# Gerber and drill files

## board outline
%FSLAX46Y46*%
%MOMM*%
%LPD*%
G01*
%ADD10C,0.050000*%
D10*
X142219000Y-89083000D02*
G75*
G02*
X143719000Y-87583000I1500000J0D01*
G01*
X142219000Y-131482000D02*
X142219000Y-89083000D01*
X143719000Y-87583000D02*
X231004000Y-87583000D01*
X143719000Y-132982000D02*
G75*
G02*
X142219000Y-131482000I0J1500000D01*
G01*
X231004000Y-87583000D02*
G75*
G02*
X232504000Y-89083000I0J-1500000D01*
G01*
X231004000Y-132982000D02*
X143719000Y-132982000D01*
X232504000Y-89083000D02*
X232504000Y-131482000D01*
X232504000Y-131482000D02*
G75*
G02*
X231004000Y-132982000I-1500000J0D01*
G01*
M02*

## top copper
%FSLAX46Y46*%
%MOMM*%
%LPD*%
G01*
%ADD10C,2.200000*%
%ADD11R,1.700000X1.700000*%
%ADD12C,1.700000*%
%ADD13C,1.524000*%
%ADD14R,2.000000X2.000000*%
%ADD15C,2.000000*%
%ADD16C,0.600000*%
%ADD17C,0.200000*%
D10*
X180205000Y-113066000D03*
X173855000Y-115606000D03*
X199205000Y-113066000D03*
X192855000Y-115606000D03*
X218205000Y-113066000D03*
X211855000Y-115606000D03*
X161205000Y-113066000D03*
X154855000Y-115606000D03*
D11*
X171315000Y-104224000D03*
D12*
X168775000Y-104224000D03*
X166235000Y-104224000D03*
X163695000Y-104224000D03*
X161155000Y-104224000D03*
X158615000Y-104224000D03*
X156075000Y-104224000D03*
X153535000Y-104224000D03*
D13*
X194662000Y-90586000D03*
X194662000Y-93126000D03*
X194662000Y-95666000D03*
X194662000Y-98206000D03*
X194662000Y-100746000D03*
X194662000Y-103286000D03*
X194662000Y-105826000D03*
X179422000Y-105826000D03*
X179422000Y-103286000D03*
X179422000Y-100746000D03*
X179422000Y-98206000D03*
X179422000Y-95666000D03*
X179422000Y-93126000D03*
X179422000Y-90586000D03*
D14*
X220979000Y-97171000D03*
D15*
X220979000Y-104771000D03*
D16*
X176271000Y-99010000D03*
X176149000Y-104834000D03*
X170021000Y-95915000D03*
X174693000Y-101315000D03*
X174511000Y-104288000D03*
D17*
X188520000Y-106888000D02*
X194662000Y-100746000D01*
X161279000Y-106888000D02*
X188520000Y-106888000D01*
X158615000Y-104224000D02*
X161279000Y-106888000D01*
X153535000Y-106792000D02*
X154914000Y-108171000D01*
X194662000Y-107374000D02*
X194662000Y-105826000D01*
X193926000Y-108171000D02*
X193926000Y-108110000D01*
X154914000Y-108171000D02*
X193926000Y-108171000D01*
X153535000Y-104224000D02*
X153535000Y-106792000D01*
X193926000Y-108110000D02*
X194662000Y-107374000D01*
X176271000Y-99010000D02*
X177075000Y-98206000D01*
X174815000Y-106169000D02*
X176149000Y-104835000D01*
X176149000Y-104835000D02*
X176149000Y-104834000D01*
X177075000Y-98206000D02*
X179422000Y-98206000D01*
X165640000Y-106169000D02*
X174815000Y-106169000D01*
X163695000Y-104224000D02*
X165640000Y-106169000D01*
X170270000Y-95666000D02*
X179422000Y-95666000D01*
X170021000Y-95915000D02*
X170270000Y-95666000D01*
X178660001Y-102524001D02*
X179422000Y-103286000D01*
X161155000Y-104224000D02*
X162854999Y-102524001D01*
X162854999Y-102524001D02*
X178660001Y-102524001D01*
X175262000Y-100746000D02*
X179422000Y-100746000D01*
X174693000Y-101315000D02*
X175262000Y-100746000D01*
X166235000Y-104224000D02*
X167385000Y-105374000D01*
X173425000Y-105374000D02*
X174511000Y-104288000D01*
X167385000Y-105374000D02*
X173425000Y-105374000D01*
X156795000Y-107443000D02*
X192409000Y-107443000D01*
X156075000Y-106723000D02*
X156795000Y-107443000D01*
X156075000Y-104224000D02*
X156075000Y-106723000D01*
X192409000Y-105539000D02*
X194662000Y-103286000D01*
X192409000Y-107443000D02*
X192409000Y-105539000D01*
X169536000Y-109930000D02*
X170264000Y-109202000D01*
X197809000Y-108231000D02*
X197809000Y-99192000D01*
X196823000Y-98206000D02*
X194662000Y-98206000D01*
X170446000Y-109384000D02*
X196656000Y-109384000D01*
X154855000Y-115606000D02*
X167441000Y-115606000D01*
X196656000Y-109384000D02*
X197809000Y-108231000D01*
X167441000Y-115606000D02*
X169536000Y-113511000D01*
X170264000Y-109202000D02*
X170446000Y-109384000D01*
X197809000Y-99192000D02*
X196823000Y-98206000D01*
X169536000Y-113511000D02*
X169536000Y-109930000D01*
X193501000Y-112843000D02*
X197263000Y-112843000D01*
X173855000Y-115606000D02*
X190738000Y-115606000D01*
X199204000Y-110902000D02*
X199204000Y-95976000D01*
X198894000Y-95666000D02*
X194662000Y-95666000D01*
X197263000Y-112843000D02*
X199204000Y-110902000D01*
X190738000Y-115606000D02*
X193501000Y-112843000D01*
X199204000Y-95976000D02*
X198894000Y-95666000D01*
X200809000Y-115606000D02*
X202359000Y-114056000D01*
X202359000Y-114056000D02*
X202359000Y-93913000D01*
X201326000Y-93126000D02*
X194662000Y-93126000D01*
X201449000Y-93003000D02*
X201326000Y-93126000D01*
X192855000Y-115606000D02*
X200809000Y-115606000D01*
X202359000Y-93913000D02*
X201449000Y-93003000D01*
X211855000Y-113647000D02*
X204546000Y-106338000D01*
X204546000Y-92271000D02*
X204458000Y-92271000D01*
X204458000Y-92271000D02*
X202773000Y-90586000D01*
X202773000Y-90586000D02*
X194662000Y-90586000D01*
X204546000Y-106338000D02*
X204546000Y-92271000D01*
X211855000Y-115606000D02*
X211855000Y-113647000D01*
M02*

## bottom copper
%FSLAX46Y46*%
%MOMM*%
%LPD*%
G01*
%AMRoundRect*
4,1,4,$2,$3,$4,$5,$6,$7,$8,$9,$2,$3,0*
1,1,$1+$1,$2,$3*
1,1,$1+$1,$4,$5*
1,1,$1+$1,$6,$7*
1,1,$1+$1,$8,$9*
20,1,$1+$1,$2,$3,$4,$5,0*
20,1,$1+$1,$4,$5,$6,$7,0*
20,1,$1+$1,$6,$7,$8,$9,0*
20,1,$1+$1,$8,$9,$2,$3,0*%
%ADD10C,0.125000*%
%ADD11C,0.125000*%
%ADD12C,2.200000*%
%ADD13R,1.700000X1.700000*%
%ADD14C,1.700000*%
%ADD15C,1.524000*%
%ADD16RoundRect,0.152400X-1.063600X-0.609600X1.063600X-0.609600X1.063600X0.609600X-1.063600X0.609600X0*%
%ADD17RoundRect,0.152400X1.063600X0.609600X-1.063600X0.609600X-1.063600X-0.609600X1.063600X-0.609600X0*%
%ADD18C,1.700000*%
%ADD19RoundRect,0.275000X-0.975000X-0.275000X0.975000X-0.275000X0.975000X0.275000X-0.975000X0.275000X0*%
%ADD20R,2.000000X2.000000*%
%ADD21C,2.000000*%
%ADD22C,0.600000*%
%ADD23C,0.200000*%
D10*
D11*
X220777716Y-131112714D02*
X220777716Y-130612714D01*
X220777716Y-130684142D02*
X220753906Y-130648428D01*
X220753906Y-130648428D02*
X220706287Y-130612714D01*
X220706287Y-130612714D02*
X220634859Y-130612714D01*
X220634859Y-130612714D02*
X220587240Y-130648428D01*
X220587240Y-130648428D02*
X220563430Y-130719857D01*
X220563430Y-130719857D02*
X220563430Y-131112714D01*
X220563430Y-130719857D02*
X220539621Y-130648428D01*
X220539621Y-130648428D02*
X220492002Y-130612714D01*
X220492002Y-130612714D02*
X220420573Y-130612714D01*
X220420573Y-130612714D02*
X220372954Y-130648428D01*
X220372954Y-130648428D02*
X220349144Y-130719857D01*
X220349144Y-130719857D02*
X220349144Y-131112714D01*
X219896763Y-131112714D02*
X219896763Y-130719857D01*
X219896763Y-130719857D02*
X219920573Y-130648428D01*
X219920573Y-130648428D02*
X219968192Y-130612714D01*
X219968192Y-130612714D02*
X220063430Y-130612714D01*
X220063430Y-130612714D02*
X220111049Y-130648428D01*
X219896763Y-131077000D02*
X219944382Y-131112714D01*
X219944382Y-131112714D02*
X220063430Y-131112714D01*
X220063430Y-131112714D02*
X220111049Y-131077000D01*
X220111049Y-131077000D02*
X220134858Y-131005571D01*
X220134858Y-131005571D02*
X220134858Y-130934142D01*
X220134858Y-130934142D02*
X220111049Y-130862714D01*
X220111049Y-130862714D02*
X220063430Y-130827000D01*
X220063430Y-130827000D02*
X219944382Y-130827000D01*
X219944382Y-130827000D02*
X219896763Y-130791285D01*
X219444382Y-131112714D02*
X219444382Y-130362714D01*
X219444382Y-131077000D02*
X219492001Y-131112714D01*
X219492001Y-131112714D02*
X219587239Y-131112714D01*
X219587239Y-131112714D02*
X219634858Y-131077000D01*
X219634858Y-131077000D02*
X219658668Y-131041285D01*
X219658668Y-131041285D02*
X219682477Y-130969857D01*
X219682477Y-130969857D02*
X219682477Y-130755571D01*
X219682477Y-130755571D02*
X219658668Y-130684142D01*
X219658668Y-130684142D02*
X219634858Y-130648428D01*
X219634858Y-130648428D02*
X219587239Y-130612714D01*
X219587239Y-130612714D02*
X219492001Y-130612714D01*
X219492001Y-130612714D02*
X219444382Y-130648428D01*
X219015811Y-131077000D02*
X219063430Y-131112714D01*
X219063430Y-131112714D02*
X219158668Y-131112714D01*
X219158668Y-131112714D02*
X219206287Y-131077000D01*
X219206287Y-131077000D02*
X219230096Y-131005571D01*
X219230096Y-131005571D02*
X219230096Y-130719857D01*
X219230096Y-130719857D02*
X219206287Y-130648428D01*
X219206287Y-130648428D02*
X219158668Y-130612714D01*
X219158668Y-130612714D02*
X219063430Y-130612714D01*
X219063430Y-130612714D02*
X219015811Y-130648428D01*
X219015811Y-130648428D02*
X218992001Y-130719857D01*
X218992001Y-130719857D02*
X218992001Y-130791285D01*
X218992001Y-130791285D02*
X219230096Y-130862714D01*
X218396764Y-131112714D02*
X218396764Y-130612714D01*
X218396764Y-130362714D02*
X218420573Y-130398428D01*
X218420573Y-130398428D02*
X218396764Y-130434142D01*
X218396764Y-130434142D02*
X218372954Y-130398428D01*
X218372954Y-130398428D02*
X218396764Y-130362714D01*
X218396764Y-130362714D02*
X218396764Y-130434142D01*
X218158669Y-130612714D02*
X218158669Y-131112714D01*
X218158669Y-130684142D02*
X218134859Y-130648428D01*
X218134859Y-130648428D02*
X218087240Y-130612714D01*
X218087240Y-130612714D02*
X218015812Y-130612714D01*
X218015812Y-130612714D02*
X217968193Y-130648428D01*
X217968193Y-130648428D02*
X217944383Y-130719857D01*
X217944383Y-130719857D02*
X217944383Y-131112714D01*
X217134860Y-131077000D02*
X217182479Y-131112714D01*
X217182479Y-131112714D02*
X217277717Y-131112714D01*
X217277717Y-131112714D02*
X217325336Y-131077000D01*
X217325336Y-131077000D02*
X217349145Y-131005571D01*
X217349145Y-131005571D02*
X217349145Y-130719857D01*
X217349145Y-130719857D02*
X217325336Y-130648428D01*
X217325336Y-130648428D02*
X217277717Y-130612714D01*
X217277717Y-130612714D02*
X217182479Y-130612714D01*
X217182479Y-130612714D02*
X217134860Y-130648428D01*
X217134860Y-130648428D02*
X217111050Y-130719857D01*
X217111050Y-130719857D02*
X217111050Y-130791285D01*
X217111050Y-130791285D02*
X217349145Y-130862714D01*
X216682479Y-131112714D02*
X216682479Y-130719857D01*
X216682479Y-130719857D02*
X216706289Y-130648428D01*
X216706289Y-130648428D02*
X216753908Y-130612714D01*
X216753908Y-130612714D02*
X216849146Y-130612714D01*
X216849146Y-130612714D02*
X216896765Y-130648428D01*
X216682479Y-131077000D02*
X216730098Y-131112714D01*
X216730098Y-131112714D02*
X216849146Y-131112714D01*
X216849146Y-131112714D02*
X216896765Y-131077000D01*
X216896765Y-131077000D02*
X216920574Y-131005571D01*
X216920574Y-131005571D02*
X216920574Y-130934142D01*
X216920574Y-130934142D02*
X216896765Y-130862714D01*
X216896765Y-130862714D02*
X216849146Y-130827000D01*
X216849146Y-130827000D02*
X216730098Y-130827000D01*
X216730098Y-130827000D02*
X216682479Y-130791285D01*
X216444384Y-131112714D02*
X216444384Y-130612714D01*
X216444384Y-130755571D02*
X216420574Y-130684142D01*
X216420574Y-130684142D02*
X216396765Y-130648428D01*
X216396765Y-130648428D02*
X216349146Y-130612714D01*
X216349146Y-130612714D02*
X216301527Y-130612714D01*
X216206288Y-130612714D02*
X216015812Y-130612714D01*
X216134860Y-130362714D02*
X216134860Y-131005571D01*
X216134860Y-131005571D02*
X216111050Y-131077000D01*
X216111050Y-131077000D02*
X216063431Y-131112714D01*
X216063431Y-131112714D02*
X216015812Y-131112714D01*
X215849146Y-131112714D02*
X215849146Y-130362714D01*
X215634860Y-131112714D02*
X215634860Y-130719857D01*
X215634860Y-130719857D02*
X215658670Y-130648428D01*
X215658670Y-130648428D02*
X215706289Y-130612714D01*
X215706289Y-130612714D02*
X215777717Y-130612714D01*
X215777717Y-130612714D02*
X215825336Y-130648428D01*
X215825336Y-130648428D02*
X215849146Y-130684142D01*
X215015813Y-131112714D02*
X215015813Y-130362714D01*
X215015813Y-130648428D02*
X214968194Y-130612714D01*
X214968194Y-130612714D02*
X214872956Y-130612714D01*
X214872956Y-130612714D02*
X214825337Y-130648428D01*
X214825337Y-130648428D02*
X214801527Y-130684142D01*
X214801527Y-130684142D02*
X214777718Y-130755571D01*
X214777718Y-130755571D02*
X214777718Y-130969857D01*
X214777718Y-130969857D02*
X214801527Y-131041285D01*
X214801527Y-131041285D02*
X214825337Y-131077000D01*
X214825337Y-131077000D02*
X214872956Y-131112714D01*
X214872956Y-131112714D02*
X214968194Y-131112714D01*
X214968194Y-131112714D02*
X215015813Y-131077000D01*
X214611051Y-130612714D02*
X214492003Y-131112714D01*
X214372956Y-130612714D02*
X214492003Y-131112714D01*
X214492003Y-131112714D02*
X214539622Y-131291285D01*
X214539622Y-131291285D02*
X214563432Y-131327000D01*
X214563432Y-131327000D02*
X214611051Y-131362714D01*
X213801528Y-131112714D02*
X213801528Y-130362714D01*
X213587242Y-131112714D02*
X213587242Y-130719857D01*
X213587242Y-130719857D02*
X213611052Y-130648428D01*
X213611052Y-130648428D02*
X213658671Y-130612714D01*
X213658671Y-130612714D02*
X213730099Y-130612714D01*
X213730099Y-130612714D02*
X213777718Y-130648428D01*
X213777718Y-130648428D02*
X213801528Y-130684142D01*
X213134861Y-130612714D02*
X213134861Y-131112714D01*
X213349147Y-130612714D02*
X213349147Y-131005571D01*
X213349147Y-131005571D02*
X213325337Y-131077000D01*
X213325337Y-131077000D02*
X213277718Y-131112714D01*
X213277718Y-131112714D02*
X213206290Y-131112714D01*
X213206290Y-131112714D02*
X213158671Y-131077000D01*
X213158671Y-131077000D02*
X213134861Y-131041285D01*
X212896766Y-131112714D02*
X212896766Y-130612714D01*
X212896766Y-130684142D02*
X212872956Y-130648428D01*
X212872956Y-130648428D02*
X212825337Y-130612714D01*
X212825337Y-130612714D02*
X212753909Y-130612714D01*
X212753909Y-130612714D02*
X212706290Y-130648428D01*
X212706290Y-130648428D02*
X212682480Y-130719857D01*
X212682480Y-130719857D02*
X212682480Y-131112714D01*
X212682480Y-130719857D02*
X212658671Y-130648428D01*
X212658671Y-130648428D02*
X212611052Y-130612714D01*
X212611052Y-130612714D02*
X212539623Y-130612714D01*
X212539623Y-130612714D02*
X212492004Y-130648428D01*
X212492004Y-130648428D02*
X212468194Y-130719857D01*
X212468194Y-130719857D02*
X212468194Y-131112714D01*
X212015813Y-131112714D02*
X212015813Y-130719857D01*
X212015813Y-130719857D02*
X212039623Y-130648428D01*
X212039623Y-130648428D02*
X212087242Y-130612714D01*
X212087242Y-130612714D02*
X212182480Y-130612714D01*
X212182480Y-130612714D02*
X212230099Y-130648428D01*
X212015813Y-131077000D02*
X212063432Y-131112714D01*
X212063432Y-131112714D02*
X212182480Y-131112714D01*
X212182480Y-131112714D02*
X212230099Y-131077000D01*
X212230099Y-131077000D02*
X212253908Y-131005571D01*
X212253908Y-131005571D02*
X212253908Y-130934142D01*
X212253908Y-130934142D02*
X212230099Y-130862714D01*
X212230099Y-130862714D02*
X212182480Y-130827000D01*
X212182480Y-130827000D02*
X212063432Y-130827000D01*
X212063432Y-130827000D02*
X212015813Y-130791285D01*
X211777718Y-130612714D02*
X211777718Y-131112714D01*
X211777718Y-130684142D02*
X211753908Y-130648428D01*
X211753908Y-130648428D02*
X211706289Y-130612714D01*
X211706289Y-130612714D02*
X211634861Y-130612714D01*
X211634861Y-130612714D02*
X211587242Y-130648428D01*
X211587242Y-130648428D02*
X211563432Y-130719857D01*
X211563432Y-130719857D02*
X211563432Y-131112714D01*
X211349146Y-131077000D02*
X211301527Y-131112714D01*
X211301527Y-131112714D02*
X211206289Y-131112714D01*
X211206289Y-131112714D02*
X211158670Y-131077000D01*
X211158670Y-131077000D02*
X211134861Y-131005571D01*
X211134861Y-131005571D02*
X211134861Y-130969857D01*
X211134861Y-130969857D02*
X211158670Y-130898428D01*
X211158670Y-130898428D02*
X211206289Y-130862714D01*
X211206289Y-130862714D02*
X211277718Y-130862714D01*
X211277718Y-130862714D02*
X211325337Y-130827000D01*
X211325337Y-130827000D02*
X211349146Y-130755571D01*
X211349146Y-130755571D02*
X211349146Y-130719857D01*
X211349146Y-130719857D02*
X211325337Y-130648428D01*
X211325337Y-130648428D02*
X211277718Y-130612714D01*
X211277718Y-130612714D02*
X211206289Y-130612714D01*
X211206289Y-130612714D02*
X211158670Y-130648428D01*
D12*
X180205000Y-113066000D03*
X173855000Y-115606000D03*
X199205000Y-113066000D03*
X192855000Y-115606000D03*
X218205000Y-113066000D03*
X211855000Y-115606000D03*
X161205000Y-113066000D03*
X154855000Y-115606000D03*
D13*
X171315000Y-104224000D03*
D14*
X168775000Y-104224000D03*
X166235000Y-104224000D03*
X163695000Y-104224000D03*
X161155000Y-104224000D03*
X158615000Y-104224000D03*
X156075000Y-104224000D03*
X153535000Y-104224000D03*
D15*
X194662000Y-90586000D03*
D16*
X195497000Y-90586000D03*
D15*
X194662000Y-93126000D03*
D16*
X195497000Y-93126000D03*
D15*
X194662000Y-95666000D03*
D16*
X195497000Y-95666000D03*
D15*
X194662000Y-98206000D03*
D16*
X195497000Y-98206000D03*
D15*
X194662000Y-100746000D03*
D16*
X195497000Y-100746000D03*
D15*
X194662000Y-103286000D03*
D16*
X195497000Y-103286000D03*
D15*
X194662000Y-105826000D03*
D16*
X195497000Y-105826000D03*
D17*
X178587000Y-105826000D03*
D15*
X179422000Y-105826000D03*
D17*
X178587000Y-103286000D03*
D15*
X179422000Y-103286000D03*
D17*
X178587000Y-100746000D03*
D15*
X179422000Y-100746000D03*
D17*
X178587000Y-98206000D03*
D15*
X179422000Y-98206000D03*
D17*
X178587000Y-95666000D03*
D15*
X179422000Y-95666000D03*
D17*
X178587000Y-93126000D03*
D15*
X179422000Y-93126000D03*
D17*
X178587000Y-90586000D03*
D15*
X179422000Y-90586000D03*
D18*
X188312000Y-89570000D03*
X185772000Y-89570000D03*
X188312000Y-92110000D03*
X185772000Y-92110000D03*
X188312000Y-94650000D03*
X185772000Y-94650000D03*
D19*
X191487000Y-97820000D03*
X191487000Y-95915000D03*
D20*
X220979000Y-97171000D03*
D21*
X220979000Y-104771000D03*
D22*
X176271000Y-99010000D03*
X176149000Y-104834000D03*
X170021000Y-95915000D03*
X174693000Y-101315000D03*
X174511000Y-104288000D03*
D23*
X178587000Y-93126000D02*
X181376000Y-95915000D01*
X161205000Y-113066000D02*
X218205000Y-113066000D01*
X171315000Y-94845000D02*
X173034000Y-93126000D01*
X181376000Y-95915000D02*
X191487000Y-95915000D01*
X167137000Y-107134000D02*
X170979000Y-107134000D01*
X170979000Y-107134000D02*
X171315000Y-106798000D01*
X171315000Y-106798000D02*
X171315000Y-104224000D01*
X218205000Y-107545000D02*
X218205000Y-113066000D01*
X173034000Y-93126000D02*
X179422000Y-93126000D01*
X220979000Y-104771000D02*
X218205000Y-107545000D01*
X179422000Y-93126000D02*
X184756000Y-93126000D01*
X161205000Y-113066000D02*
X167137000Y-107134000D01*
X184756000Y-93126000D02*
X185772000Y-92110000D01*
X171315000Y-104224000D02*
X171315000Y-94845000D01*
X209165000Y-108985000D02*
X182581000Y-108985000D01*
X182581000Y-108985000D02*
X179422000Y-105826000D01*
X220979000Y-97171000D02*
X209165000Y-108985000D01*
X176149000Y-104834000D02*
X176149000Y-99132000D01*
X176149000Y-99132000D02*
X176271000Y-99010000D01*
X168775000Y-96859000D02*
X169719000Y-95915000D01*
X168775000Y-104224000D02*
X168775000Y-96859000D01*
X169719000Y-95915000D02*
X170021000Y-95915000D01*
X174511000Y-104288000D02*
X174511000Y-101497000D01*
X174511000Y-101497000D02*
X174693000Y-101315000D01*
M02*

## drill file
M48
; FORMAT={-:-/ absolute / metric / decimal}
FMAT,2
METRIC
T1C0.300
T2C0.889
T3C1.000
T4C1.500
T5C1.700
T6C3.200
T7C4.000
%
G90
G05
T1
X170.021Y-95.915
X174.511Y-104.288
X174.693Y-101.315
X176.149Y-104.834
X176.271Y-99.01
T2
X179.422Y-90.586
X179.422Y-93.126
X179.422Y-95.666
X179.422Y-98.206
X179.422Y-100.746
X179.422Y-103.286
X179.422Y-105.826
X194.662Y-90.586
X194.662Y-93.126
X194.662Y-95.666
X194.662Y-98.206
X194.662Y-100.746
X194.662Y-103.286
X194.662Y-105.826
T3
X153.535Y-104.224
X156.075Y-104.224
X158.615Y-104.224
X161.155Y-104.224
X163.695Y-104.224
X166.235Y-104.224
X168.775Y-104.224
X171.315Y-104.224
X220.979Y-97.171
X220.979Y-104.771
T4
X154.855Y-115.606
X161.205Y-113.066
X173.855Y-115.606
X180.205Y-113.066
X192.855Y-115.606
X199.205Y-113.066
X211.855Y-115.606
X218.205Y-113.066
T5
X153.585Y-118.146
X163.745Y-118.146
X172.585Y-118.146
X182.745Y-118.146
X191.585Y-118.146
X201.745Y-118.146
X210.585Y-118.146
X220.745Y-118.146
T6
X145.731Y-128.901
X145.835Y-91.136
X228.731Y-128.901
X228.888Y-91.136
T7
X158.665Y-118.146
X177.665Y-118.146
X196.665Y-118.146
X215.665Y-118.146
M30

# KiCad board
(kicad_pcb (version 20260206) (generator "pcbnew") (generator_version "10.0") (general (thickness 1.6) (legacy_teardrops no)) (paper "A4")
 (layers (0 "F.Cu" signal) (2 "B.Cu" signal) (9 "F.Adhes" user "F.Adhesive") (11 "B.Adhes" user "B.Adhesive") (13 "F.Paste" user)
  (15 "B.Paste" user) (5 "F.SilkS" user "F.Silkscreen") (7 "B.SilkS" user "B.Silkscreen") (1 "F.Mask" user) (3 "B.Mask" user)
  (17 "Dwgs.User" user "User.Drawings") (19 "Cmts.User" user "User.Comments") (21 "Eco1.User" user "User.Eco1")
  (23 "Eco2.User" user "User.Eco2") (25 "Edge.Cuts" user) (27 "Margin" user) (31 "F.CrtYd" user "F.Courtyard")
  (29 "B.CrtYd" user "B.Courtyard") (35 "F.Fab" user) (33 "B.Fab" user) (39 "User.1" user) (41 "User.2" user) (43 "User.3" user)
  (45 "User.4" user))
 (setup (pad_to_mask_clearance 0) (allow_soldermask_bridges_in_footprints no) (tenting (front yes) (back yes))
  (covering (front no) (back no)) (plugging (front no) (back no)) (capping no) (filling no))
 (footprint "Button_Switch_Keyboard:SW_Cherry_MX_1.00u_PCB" (layer "F.Cu") (at 180.205 113.066)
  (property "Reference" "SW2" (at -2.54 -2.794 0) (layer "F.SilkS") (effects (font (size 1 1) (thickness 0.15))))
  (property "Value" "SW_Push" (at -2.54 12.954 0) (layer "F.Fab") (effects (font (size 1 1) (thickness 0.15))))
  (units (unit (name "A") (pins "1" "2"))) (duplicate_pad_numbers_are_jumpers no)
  (pad "" np_thru_hole circle (at -7.62 5.08) (size 1.7 1.7) (drill 1.7) (layers "*.Cu" "*.Mask"))
  (pad "" np_thru_hole circle (at -2.54 5.08) (size 4 4) (drill 4) (layers "*.Cu" "*.Mask"))
  (pad "" np_thru_hole circle (at 2.54 5.08) (size 1.7 1.7) (drill 1.7) (layers "*.Cu" "*.Mask"))
  (pad "1" thru_hole circle (at 0 0) (size 2.2 2.2) (drill 1.5) (layers "*.Cu" "*.Mask") (remove_unused_layers no) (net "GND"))
  (pad "2" thru_hole circle (at -6.35 2.54) (size 2.2 2.2) (drill 1.5) (layers "*.Cu" "*.Mask") (remove_unused_layers no)
   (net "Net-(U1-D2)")))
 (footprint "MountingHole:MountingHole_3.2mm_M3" (layer "F.Cu") (at 228.888 91.136)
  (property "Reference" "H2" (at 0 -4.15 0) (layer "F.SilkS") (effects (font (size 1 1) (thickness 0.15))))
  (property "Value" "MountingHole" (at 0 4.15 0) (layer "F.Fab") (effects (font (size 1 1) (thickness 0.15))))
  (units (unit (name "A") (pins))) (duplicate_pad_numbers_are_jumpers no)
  (pad "" np_thru_hole circle (at 0 0) (size 3.2 3.2) (drill 3.2) (layers "*.Cu" "*.Mask")))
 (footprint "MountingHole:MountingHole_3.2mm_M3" (layer "F.Cu") (at 145.731 128.901)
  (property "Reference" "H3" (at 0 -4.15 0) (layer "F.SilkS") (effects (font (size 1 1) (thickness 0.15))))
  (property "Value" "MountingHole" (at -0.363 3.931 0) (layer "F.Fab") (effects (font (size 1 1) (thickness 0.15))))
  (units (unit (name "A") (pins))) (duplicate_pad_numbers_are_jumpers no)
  (pad "" np_thru_hole circle (at 0 0) (size 3.2 3.2) (drill 3.2) (layers "*.Cu" "*.Mask")))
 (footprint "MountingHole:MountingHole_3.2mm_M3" (layer "F.Cu") (at 228.731 128.901)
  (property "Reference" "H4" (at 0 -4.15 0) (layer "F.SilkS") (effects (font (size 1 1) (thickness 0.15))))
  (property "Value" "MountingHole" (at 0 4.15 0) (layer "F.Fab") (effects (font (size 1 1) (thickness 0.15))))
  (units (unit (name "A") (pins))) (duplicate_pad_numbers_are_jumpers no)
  (pad "" np_thru_hole circle (at 0 0) (size 3.2 3.2) (drill 3.2) (layers "*.Cu" "*.Mask")))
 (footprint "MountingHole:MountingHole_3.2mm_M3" (layer "F.Cu") (at 145.835 91.136)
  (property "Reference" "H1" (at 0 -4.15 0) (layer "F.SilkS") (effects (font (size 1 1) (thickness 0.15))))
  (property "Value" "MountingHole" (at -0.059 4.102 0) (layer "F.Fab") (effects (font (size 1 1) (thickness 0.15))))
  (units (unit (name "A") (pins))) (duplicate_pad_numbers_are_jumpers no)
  (pad "" np_thru_hole circle (at 0 0) (size 3.2 3.2) (drill 3.2) (layers "*.Cu" "*.Mask")))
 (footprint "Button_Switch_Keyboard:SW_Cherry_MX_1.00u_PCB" (layer "F.Cu") (at 199.205 113.066)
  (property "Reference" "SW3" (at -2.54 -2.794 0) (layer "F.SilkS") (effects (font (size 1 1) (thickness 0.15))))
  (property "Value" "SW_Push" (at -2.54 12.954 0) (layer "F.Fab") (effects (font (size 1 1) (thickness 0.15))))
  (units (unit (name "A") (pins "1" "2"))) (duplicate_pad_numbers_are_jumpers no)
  (pad "" np_thru_hole circle (at -7.62 5.08) (size 1.7 1.7) (drill 1.7) (layers "*.Cu" "*.Mask"))
  (pad "" np_thru_hole circle (at -2.54 5.08) (size 4 4) (drill 4) (layers "*.Cu" "*.Mask"))
  (pad "" np_thru_hole circle (at 2.54 5.08) (size 1.7 1.7) (drill 1.7) (layers "*.Cu" "*.Mask"))
  (pad "1" thru_hole circle (at 0 0) (size 2.2 2.2) (drill 1.5) (layers "*.Cu" "*.Mask") (remove_unused_layers no) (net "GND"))
  (pad "2" thru_hole circle (at -6.35 2.54) (size 2.2 2.2) (drill 1.5) (layers "*.Cu" "*.Mask") (remove_unused_layers no)
   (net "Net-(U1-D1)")))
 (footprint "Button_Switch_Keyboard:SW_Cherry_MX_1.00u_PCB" (layer "F.Cu") (at 218.205 113.066)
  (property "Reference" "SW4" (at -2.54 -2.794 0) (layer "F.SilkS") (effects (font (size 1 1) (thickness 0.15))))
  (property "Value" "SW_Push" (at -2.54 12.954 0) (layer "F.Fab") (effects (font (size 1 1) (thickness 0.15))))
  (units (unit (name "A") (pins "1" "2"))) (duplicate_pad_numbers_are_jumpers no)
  (pad "" np_thru_hole circle (at -7.62 5.08) (size 1.7 1.7) (drill 1.7) (layers "*.Cu" "*.Mask"))
  (pad "" np_thru_hole circle (at -2.54 5.08) (size 4 4) (drill 4) (layers "*.Cu" "*.Mask"))
  (pad "" np_thru_hole circle (at 2.54 5.08) (size 1.7 1.7) (drill 1.7) (layers "*.Cu" "*.Mask"))
  (pad "1" thru_hole circle (at 0 0) (size 2.2 2.2) (drill 1.5) (layers "*.Cu" "*.Mask") (remove_unused_layers no) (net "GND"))
  (pad "2" thru_hole circle (at -6.35 2.54) (size 2.2 2.2) (drill 1.5) (layers "*.Cu" "*.Mask") (remove_unused_layers no)
   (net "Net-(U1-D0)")))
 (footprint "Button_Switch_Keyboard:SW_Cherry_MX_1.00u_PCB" (layer "F.Cu") (at 161.205 113.066)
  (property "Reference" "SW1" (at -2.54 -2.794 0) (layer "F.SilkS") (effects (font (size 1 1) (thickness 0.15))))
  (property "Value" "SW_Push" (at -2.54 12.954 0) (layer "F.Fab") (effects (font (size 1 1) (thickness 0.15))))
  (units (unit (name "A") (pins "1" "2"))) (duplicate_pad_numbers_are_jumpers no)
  (pad "" np_thru_hole circle (at -7.62 5.08) (size 1.7 1.7) (drill 1.7) (layers "*.Cu" "*.Mask"))
  (pad "" np_thru_hole circle (at -2.54 5.08) (size 4 4) (drill 4) (layers "*.Cu" "*.Mask"))
  (pad "" np_thru_hole circle (at 2.54 5.08) (size 1.7 1.7) (drill 1.7) (layers "*.Cu" "*.Mask"))
  (pad "1" thru_hole circle (at 0 0) (size 2.2 2.2) (drill 1.5) (layers "*.Cu" "*.Mask") (remove_unused_layers no) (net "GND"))
  (pad "2" thru_hole circle (at -6.35 2.54) (size 2.2 2.2) (drill 1.5) (layers "*.Cu" "*.Mask") (remove_unused_layers no)
   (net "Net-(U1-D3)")))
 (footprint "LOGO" (layer "F.Cu") (at 158.714 92.166)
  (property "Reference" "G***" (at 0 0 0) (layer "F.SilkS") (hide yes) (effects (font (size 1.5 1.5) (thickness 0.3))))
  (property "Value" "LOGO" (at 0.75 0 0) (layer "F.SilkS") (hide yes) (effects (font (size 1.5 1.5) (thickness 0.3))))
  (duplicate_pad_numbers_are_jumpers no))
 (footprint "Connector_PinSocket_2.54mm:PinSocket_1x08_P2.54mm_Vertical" (layer "B.Cu") (at 171.315 104.224 90)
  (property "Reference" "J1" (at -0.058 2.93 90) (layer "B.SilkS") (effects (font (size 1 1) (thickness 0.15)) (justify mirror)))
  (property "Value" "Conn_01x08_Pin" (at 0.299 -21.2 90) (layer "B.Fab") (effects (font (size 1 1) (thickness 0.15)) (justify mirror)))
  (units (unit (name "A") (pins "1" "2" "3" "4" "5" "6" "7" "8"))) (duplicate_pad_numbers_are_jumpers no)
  (pad "1" thru_hole rect (at 0 0 90) (size 1.7 1.7) (drill 1) (layers "*.Cu" "*.Mask") (remove_unused_layers no) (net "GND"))
  (pad "2" thru_hole circle (at 0 -2.54 90) (size 1.7 1.7) (drill 1) (layers "*.Cu" "*.Mask") (remove_unused_layers no) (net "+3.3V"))
  (pad "3" thru_hole circle (at 0 -5.08 90) (size 1.7 1.7) (drill 1) (layers "*.Cu" "*.Mask") (remove_unused_layers no) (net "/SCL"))
  (pad "4" thru_hole circle (at 0 -7.62 90) (size 1.7 1.7) (drill 1) (layers "*.Cu" "*.Mask") (remove_unused_layers no) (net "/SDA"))
  (pad "5" thru_hole circle (at 0 -10.16 90) (size 1.7 1.7) (drill 1) (layers "*.Cu" "*.Mask") (remove_unused_layers no) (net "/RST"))
  (pad "6" thru_hole circle (at 0 -12.7 90) (size 1.7 1.7) (drill 1) (layers "*.Cu" "*.Mask") (remove_unused_layers no) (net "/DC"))
  (pad "7" thru_hole circle (at 0 -15.24 90) (size 1.7 1.7) (drill 1) (layers "*.Cu" "*.Mask") (remove_unused_layers no) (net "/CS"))
  (pad "8" thru_hole circle (at 0 -17.78 90) (size 1.7 1.7) (drill 1) (layers "*.Cu" "*.Mask") (remove_unused_layers no) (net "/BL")))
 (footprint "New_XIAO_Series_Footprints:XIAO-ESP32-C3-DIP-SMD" (layer "B.Cu") (at 187.042 98.206 90)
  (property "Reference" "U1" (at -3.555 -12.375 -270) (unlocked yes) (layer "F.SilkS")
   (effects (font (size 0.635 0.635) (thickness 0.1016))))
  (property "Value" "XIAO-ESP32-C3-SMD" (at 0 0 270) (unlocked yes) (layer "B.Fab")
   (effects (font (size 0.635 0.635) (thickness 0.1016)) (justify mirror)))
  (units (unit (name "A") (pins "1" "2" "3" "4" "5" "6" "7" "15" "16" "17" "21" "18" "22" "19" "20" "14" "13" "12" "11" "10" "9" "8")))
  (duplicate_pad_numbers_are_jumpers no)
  (pad "1" thru_hole circle (at 7.62 7.62) (size 1.524 1.524) (drill 0.889) (layers "*.Cu" "*.Mask") (remove_unused_layers no)
   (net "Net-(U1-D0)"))
  (pad "1" smd roundrect (at 7.62 8.455) (size 2.432 1.524) (layers "B.Cu" "B.Mask") (roundrect_rratio 0.1) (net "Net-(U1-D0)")
   (thermal_bridge_angle 45))
  (pad "2" thru_hole circle (at 5.08 7.62) (size 1.524 1.524) (drill 0.889) (layers "*.Cu" "*.Mask") (remove_unused_layers no)
   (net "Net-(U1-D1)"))
  (pad "2" smd roundrect (at 5.08 8.455) (size 2.432 1.524) (layers "B.Cu" "B.Mask") (roundrect_rratio 0.1) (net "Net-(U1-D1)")
   (thermal_bridge_angle 45))
  (pad "3" thru_hole circle (at 2.54 7.62) (size 1.524 1.524) (drill 0.889) (layers "*.Cu" "*.Mask") (remove_unused_layers no)
   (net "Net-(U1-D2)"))
  (pad "3" smd roundrect (at 2.54 8.455) (size 2.432 1.524) (layers "B.Cu" "B.Mask") (roundrect_rratio 0.1) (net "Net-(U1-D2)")
   (thermal_bridge_angle 45))
  (pad "4" thru_hole circle (at 0 7.62) (size 1.524 1.524) (drill 0.889) (layers "*.Cu" "*.Mask") (remove_unused_layers no)
   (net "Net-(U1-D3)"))
  (pad "4" smd roundrect (at 0 8.455) (size 2.432 1.524) (layers "B.Cu" "B.Mask") (roundrect_rratio 0.1) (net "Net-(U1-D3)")
   (thermal_bridge_angle 45))
  (pad "5" thru_hole circle (at -2.54 7.62) (size 1.524 1.524) (drill 0.889) (layers "*.Cu" "*.Mask") (remove_unused_layers no) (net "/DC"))
  (pad "5" smd roundrect (at -2.54 8.455) (size 2.432 1.524) (layers "B.Cu" "B.Mask") (roundrect_rratio 0.1) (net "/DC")
   (thermal_bridge_angle 45))
  (pad "6" thru_hole circle (at -5.08 7.62) (size 1.524 1.524) (drill 0.889) (layers "*.Cu" "*.Mask") (remove_unused_layers no) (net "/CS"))
  (pad "6" smd roundrect (at -5.08 8.455) (size 2.432 1.524) (layers "B.Cu" "B.Mask") (roundrect_rratio 0.1) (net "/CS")
   (thermal_bridge_angle 45))
  (pad "7" thru_hole circle (at -7.62 7.62) (size 1.524 1.524) (drill 0.889) (layers "*.Cu" "*.Mask") (remove_unused_layers no) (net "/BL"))
  (pad "7" smd roundrect (at -7.62 8.455) (size 2.432 1.524) (layers "B.Cu" "B.Mask") (roundrect_rratio 0.1) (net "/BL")
   (thermal_bridge_angle 45))
  (pad "8" smd roundrect (at -7.62 -8.455 180) (size 2.432 1.524) (layers "B.Cu" "B.Mask") (roundrect_rratio 0.1) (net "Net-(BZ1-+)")
   (thermal_bridge_angle 45))
  (pad "8" thru_hole circle (at -7.62 -7.62 180) (size 1.524 1.524) (drill 0.889) (layers "*.Cu" "*.Mask") (remove_unused_layers no)
   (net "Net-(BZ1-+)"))
  (pad "9" smd roundrect (at -5.08 -8.455 180) (size 2.432 1.524) (layers "B.Cu" "B.Mask") (roundrect_rratio 0.1) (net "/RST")
   (thermal_bridge_angle 45))
  (pad "9" thru_hole circle (at -5.08 -7.62 180) (size 1.524 1.524) (drill 0.889) (layers "*.Cu" "*.Mask") (remove_unused_layers no)
   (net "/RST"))
  (pad "10" smd roundrect (at -2.54 -8.455 180) (size 2.432 1.524) (layers "B.Cu" "B.Mask") (roundrect_rratio 0.1) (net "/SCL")
   (thermal_bridge_angle 45))
  (pad "10" thru_hole circle (at -2.54 -7.62 180) (size 1.524 1.524) (drill 0.889) (layers "*.Cu" "*.Mask") (remove_unused_layers no)
   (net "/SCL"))
  (pad "11" smd roundrect (at 0 -8.455 180) (size 2.432 1.524) (layers "B.Cu" "B.Mask") (roundrect_rratio 0.1) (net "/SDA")
   (thermal_bridge_angle 45))
  (pad "11" thru_hole circle (at 0 -7.62 180) (size 1.524 1.524) (drill 0.889) (layers "*.Cu" "*.Mask") (remove_unused_layers no)
   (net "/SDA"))
  (pad "12" smd roundrect (at 2.54 -8.455 180) (size 2.432 1.524) (layers "B.Cu" "B.Mask") (roundrect_rratio 0.1) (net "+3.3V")
   (thermal_bridge_angle 45))
  (pad "12" thru_hole circle (at 2.54 -7.62 180) (size 1.524 1.524) (drill 0.889) (layers "*.Cu" "*.Mask") (remove_unused_layers no)
   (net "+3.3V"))
  (pad "13" smd roundrect (at 5.08 -8.455 180) (size 2.432 1.524) (layers "B.Cu" "B.Mask") (roundrect_rratio 0.1) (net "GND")
   (thermal_bridge_angle 45))
  (pad "13" thru_hole circle (at 5.08 -7.62 180) (size 1.524 1.524) (drill 0.889) (layers "*.Cu" "*.Mask") (remove_unused_layers no)
   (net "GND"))
  (pad "14" smd roundrect (at 7.62 -8.455 180) (size 2.432 1.524) (layers "B.Cu" "B.Mask") (roundrect_rratio 0.1)
   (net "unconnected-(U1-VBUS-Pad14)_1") (thermal_bridge_angle 45))
  (pad "14" thru_hole circle (at 7.62 -7.62 180) (size 1.524 1.524) (drill 0.889) (layers "*.Cu" "*.Mask") (remove_unused_layers no)
   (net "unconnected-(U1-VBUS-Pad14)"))
  (pad "15" smd circle (at 8.636 1.27 180) (size 1.7 1.7) (layers "B.Cu" "B.Mask" "B.Paste") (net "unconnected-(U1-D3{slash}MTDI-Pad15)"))
  (pad "16" smd circle (at 8.636 -1.27 180) (size 1.7 1.7) (layers "B.Cu" "B.Mask" "B.Paste") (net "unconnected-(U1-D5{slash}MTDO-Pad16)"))
  (pad "17" smd circle (at 6.096 1.27 180) (size 1.7 1.7) (layers "B.Cu" "B.Mask" "B.Paste") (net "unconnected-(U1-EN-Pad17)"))
  (pad "18" smd circle (at 6.096 -1.27 180) (size 1.7 1.7) (layers "B.Cu" "B.Mask" "B.Paste") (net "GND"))
  (pad "19" smd circle (at 3.556 1.27 180) (size 1.7 1.7) (layers "B.Cu" "B.Mask" "B.Paste") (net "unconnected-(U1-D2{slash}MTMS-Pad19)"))
  (pad "20" smd circle (at 3.556 -1.27 180) (size 1.7 1.7) (layers "B.Cu" "B.Mask" "B.Paste") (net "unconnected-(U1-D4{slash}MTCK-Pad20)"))
  (pad "21" smd roundrect (at 0.386 4.445) (size 2.5 1.1) (layers "B.Cu" "B.Mask" "B.Paste") (roundrect_rratio 0.25)
   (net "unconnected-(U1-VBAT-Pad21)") (thermal_bridge_angle 45))
  (pad "22" smd roundrect (at 2.291 4.445) (size 2.5 1.1) (layers "B.Cu" "B.Mask" "B.Paste") (roundrect_rratio 0.25) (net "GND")
   (thermal_bridge_angle 45)))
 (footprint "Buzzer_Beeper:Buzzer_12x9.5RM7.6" (layer "B.Cu") (at 220.979 97.171 -90)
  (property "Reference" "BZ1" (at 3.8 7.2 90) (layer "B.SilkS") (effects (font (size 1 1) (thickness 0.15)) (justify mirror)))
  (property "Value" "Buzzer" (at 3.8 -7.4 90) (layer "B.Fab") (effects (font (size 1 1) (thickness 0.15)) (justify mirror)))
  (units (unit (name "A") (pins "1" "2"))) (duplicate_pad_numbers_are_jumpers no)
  (pad "1" thru_hole rect (at 0 0 270) (size 2 2) (drill 1) (layers "*.Cu" "*.Mask") (remove_unused_layers no) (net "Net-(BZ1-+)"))
  (pad "2" thru_hole circle (at 7.6 0 270) (size 2 2) (drill 1) (layers "*.Cu" "*.Mask") (remove_unused_layers no) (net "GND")))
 (gr_arc (start 142.219 89.083) (mid 142.65834 88.02234) (end 143.719 87.583) (stroke (width 0.05) (type default)) (layer "Edge.Cuts"))
 (gr_line (start 142.219 131.482) (end 142.219 89.083) (stroke (width 0.05) (type default)) (layer "Edge.Cuts"))
 (gr_line (start 143.719 87.583) (end 231.004 87.583) (stroke (width 0.05) (type default)) (layer "Edge.Cuts"))
 (gr_arc (start 143.719 132.982) (mid 142.65834 132.54266) (end 142.219 131.482) (stroke (width 0.05) (type default)) (layer "Edge.Cuts"))
 (gr_arc (start 231.004 87.583) (mid 232.06466 88.02234) (end 232.504 89.083) (stroke (width 0.05) (type default)) (layer "Edge.Cuts"))
 (gr_line (start 231.004 132.982) (end 143.719 132.982) (stroke (width 0.05) (type default)) (layer "Edge.Cuts"))
 (gr_line (start 232.504 89.083) (end 232.504 131.482) (stroke (width 0.05) (type default)) (layer "Edge.Cuts"))
 (gr_arc (start 232.504 131.482) (mid 232.06466 132.54266) (end 231.004 132.982) (stroke (width 0.05) (type default)) (layer "Edge.Cuts"))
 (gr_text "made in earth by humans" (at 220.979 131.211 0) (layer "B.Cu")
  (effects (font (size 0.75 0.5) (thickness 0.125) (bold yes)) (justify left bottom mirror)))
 (segment (start 178.587 93.126) (end 181.376 95.915) (width 0.2) (layer "B.Cu") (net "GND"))
 (segment (start 161.205 113.066) (end 218.205 113.066) (width 0.2) (layer "B.Cu") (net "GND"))
 (segment (start 171.315 94.845) (end 173.034 93.126) (width 0.2) (layer "B.Cu") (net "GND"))
 (segment (start 181.376 95.915) (end 191.487 95.915) (width 0.2) (layer "B.Cu") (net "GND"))
 (segment (start 167.137 107.134) (end 170.979 107.134) (width 0.2) (layer "B.Cu") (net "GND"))
 (segment (start 170.979 107.134) (end 171.315 106.798) (width 0.2) (layer "B.Cu") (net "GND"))
 (segment (start 171.315 106.798) (end 171.315 104.224) (width 0.2) (layer "B.Cu") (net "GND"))
 (segment (start 218.205 107.545) (end 218.205 113.066) (width 0.2) (layer "B.Cu") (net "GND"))
 (segment (start 173.034 93.126) (end 179.422 93.126) (width 0.2) (layer "B.Cu") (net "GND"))
 (segment (start 220.979 104.771) (end 218.205 107.545) (width 0.2) (layer "B.Cu") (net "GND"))
 (segment (start 179.422 93.126) (end 184.756 93.126) (width 0.2) (layer "B.Cu") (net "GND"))
 (segment (start 161.205 113.066) (end 167.137 107.134) (width 0.2) (layer "B.Cu") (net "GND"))
 (segment (start 184.756 93.126) (end 185.772 92.11) (width 0.2) (layer "B.Cu") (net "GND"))
 (segment (start 171.315 104.224) (end 171.315 94.845) (width 0.2) (layer "B.Cu") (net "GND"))
 (segment (start 209.165 108.985) (end 182.581 108.985) (width 0.2) (layer "B.Cu") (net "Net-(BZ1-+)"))
 (segment (start 182.581 108.985) (end 179.422 105.826) (width 0.2) (layer "B.Cu") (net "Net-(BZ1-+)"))
 (segment (start 220.979 97.171) (end 209.165 108.985) (width 0.2) (layer "B.Cu") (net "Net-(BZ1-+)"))
 (segment (start 188.52 106.888) (end 194.662 100.746) (width 0.2) (layer "F.Cu") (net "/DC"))
 (segment (start 161.279 106.888) (end 188.52 106.888) (width 0.2) (layer "F.Cu") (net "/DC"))
 (segment (start 158.615 104.224) (end 161.279 106.888) (width 0.2) (layer "F.Cu") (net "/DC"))
 (segment (start 153.535 106.792) (end 154.914 108.171) (width 0.2) (layer "F.Cu") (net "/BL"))
 (segment (start 194.662 107.374) (end 194.662 105.826) (width 0.2) (layer "F.Cu") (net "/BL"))
 (segment (start 193.926 108.171) (end 193.926 108.11) (width 0.2) (layer "F.Cu") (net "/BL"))
 (segment (start 154.914 108.171) (end 193.926 108.171) (width 0.2) (layer "F.Cu") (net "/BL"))
 (segment (start 153.535 104.224) (end 153.535 106.792) (width 0.2) (layer "F.Cu") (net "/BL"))
 (segment (start 193.926 108.11) (end 194.662 107.374) (width 0.2) (layer "F.Cu") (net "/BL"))
 (segment (start 176.271 99.01) (end 177.075 98.206) (width 0.2) (layer "F.Cu") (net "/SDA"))
 (segment (start 174.815 106.169) (end 176.149 104.835) (width 0.2) (layer "F.Cu") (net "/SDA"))
 (segment (start 176.149 104.835) (end 176.149 104.834) (width 0.2) (layer "F.Cu") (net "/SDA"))
 (segment (start 177.075 98.206) (end 179.422 98.206) (width 0.2) (layer "F.Cu") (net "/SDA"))
 (segment (start 165.64 106.169) (end 174.815 106.169) (width 0.2) (layer "F.Cu") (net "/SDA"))
 (segment (start 163.695 104.224) (end 165.64 106.169) (width 0.2) (layer "F.Cu") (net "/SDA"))
 (via (at 176.271 99.01) (size 0.6) (drill 0.3) (layers "F.Cu" "B.Cu") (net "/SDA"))
 (via (at 176.149 104.834) (size 0.6) (drill 0.3) (layers "F.Cu" "B.Cu") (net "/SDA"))
 (segment (start 176.149 104.834) (end 176.149 99.132) (width 0.2) (layer "B.Cu") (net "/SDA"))
 (segment (start 176.149 99.132) (end 176.271 99.01) (width 0.2) (layer "B.Cu") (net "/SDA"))
 (segment (start 170.27 95.666) (end 179.422 95.666) (width 0.2) (layer "F.Cu") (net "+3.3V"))
 (segment (start 170.021 95.915) (end 170.27 95.666) (width 0.2) (layer "F.Cu") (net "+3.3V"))
 (via (at 170.021 95.915) (size 0.6) (drill 0.3) (layers "F.Cu" "B.Cu") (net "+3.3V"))
 (segment (start 168.775 96.859) (end 169.719 95.915) (width 0.2) (layer "B.Cu") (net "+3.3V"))
 (segment (start 168.775 104.224) (end 168.775 96.859) (width 0.2) (layer "B.Cu") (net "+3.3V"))
 (segment (start 169.719 95.915) (end 170.021 95.915) (width 0.2) (layer "B.Cu") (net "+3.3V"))
 (segment (start 178.660001 102.524001) (end 179.422 103.286) (width 0.2) (layer "F.Cu") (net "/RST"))
 (segment (start 161.155 104.224) (end 162.854999 102.524001) (width 0.2) (layer "F.Cu") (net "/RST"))
 (segment (start 162.854999 102.524001) (end 178.660001 102.524001) (width 0.2) (layer "F.Cu") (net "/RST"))
 (segment (start 175.262 100.746) (end 179.422 100.746) (width 0.2) (layer "F.Cu") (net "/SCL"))
 (segment (start 174.693 101.315) (end 175.262 100.746) (width 0.2) (layer "F.Cu") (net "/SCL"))
 (segment (start 166.235 104.224) (end 167.385 105.374) (width 0.2) (layer "F.Cu") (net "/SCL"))
 (segment (start 173.425 105.374) (end 174.511 104.288) (width 0.2) (layer "F.Cu") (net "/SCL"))
 (segment (start 167.385 105.374) (end 173.425 105.374) (width 0.2) (layer "F.Cu") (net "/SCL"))
 (via (at 174.693 101.315) (size 0.6) (drill 0.3) (layers "F.Cu" "B.Cu") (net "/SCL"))
 (via (at 174.511 104.288) (size 0.6) (drill 0.3) (layers "F.Cu" "B.Cu") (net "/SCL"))
 (segment (start 174.511 104.288) (end 174.511 101.497) (width 0.2) (layer "B.Cu") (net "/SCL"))
 (segment (start 174.511 101.497) (end 174.693 101.315) (width 0.2) (layer "B.Cu") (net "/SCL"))
 (segment (start 156.795 107.443) (end 192.409 107.443) (width 0.2) (layer "F.Cu") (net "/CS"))
 (segment (start 156.075 106.723) (end 156.795 107.443) (width 0.2) (layer "F.Cu") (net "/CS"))
 (segment (start 156.075 104.224) (end 156.075 106.723) (width 0.2) (layer "F.Cu") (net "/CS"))
 (segment (start 192.409 105.539) (end 194.662 103.286) (width 0.2) (layer "F.Cu") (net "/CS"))
 (segment (start 192.409 107.443) (end 192.409 105.539) (width 0.2) (layer "F.Cu") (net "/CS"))
 (segment (start 169.536 109.93) (end 170.264 109.202) (width 0.2) (layer "F.Cu") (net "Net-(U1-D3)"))
 (segment (start 197.809 108.231) (end 197.809 99.192) (width 0.2) (layer "F.Cu") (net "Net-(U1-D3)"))
 (segment (start 196.823 98.206) (end 194.662 98.206) (width 0.2) (layer "F.Cu") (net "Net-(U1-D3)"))
 (segment (start 170.446 109.384) (end 196.656 109.384) (width 0.2) (layer "F.Cu") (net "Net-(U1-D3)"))
 (segment (start 154.855 115.606) (end 167.441 115.606) (width 0.2) (layer "F.Cu") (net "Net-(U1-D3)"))
 (segment (start 196.656 109.384) (end 197.809 108.231) (width 0.2) (layer "F.Cu") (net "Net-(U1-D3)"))
 (segment (start 167.441 115.606) (end 169.536 113.511) (width 0.2) (layer "F.Cu") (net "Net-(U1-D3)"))
 (segment (start 170.264 109.202) (end 170.446 109.384) (width 0.2) (layer "F.Cu") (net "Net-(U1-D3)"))
 (segment (start 197.809 99.192) (end 196.823 98.206) (width 0.2) (layer "F.Cu") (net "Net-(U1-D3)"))
 (segment (start 169.536 113.511) (end 169.536 109.93) (width 0.2) (layer "F.Cu") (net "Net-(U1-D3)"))
 (segment (start 193.501 112.843) (end 197.263 112.843) (width 0.2) (layer "F.Cu") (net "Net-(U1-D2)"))
 (segment (start 173.855 115.606) (end 190.738 115.606) (width 0.2) (layer "F.Cu") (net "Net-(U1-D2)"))
 (segment (start 199.204 110.902) (end 199.204 95.976) (width 0.2) (layer "F.Cu") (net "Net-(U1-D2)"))
 (segment (start 198.894 95.666) (end 194.662 95.666) (width 0.2) (layer "F.Cu") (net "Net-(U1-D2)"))
 (segment (start 197.263 112.843) (end 199.204 110.902) (width 0.2) (layer "F.Cu") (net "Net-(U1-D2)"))
 (segment (start 190.738 115.606) (end 193.501 112.843) (width 0.2) (layer "F.Cu") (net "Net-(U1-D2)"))
 (segment (start 199.204 95.976) (end 198.894 95.666) (width 0.2) (layer "F.Cu") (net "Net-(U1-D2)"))
 (segment (start 200.809 115.606) (end 202.359 114.056) (width 0.2) (layer "F.Cu") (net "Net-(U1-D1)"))
 (segment (start 202.359 114.056) (end 202.359 93.913) (width 0.2) (layer "F.Cu") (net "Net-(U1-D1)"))
 (segment (start 201.326 93.126) (end 194.662 93.126) (width 0.2) (layer "F.Cu") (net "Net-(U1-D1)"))
 (segment (start 201.449 93.003) (end 201.326 93.126) (width 0.2) (layer "F.Cu") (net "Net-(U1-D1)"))
 (segment (start 192.855 115.606) (end 200.809 115.606) (width 0.2) (layer "F.Cu") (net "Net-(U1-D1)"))
 (segment (start 202.359 93.913) (end 201.449 93.003) (width 0.2) (layer "F.Cu") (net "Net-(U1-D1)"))
 (segment (start 211.855 113.647) (end 204.546 106.338) (width 0.2) (layer "F.Cu") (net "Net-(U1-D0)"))
 (segment (start 204.546 92.271) (end 204.458 92.271) (width 0.2) (layer "F.Cu") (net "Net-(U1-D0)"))
 (segment (start 204.458 92.271) (end 202.773 90.586) (width 0.2) (layer "F.Cu") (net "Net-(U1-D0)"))
 (segment (start 202.773 90.586) (end 194.662 90.586) (width 0.2) (layer "F.Cu") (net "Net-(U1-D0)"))
 (segment (start 204.546 106.338) (end 204.546 92.271) (width 0.2) (layer "F.Cu") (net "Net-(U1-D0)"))
 (segment (start 211.855 115.606) (end 211.855 113.647) (width 0.2) (layer "F.Cu") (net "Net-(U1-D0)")))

